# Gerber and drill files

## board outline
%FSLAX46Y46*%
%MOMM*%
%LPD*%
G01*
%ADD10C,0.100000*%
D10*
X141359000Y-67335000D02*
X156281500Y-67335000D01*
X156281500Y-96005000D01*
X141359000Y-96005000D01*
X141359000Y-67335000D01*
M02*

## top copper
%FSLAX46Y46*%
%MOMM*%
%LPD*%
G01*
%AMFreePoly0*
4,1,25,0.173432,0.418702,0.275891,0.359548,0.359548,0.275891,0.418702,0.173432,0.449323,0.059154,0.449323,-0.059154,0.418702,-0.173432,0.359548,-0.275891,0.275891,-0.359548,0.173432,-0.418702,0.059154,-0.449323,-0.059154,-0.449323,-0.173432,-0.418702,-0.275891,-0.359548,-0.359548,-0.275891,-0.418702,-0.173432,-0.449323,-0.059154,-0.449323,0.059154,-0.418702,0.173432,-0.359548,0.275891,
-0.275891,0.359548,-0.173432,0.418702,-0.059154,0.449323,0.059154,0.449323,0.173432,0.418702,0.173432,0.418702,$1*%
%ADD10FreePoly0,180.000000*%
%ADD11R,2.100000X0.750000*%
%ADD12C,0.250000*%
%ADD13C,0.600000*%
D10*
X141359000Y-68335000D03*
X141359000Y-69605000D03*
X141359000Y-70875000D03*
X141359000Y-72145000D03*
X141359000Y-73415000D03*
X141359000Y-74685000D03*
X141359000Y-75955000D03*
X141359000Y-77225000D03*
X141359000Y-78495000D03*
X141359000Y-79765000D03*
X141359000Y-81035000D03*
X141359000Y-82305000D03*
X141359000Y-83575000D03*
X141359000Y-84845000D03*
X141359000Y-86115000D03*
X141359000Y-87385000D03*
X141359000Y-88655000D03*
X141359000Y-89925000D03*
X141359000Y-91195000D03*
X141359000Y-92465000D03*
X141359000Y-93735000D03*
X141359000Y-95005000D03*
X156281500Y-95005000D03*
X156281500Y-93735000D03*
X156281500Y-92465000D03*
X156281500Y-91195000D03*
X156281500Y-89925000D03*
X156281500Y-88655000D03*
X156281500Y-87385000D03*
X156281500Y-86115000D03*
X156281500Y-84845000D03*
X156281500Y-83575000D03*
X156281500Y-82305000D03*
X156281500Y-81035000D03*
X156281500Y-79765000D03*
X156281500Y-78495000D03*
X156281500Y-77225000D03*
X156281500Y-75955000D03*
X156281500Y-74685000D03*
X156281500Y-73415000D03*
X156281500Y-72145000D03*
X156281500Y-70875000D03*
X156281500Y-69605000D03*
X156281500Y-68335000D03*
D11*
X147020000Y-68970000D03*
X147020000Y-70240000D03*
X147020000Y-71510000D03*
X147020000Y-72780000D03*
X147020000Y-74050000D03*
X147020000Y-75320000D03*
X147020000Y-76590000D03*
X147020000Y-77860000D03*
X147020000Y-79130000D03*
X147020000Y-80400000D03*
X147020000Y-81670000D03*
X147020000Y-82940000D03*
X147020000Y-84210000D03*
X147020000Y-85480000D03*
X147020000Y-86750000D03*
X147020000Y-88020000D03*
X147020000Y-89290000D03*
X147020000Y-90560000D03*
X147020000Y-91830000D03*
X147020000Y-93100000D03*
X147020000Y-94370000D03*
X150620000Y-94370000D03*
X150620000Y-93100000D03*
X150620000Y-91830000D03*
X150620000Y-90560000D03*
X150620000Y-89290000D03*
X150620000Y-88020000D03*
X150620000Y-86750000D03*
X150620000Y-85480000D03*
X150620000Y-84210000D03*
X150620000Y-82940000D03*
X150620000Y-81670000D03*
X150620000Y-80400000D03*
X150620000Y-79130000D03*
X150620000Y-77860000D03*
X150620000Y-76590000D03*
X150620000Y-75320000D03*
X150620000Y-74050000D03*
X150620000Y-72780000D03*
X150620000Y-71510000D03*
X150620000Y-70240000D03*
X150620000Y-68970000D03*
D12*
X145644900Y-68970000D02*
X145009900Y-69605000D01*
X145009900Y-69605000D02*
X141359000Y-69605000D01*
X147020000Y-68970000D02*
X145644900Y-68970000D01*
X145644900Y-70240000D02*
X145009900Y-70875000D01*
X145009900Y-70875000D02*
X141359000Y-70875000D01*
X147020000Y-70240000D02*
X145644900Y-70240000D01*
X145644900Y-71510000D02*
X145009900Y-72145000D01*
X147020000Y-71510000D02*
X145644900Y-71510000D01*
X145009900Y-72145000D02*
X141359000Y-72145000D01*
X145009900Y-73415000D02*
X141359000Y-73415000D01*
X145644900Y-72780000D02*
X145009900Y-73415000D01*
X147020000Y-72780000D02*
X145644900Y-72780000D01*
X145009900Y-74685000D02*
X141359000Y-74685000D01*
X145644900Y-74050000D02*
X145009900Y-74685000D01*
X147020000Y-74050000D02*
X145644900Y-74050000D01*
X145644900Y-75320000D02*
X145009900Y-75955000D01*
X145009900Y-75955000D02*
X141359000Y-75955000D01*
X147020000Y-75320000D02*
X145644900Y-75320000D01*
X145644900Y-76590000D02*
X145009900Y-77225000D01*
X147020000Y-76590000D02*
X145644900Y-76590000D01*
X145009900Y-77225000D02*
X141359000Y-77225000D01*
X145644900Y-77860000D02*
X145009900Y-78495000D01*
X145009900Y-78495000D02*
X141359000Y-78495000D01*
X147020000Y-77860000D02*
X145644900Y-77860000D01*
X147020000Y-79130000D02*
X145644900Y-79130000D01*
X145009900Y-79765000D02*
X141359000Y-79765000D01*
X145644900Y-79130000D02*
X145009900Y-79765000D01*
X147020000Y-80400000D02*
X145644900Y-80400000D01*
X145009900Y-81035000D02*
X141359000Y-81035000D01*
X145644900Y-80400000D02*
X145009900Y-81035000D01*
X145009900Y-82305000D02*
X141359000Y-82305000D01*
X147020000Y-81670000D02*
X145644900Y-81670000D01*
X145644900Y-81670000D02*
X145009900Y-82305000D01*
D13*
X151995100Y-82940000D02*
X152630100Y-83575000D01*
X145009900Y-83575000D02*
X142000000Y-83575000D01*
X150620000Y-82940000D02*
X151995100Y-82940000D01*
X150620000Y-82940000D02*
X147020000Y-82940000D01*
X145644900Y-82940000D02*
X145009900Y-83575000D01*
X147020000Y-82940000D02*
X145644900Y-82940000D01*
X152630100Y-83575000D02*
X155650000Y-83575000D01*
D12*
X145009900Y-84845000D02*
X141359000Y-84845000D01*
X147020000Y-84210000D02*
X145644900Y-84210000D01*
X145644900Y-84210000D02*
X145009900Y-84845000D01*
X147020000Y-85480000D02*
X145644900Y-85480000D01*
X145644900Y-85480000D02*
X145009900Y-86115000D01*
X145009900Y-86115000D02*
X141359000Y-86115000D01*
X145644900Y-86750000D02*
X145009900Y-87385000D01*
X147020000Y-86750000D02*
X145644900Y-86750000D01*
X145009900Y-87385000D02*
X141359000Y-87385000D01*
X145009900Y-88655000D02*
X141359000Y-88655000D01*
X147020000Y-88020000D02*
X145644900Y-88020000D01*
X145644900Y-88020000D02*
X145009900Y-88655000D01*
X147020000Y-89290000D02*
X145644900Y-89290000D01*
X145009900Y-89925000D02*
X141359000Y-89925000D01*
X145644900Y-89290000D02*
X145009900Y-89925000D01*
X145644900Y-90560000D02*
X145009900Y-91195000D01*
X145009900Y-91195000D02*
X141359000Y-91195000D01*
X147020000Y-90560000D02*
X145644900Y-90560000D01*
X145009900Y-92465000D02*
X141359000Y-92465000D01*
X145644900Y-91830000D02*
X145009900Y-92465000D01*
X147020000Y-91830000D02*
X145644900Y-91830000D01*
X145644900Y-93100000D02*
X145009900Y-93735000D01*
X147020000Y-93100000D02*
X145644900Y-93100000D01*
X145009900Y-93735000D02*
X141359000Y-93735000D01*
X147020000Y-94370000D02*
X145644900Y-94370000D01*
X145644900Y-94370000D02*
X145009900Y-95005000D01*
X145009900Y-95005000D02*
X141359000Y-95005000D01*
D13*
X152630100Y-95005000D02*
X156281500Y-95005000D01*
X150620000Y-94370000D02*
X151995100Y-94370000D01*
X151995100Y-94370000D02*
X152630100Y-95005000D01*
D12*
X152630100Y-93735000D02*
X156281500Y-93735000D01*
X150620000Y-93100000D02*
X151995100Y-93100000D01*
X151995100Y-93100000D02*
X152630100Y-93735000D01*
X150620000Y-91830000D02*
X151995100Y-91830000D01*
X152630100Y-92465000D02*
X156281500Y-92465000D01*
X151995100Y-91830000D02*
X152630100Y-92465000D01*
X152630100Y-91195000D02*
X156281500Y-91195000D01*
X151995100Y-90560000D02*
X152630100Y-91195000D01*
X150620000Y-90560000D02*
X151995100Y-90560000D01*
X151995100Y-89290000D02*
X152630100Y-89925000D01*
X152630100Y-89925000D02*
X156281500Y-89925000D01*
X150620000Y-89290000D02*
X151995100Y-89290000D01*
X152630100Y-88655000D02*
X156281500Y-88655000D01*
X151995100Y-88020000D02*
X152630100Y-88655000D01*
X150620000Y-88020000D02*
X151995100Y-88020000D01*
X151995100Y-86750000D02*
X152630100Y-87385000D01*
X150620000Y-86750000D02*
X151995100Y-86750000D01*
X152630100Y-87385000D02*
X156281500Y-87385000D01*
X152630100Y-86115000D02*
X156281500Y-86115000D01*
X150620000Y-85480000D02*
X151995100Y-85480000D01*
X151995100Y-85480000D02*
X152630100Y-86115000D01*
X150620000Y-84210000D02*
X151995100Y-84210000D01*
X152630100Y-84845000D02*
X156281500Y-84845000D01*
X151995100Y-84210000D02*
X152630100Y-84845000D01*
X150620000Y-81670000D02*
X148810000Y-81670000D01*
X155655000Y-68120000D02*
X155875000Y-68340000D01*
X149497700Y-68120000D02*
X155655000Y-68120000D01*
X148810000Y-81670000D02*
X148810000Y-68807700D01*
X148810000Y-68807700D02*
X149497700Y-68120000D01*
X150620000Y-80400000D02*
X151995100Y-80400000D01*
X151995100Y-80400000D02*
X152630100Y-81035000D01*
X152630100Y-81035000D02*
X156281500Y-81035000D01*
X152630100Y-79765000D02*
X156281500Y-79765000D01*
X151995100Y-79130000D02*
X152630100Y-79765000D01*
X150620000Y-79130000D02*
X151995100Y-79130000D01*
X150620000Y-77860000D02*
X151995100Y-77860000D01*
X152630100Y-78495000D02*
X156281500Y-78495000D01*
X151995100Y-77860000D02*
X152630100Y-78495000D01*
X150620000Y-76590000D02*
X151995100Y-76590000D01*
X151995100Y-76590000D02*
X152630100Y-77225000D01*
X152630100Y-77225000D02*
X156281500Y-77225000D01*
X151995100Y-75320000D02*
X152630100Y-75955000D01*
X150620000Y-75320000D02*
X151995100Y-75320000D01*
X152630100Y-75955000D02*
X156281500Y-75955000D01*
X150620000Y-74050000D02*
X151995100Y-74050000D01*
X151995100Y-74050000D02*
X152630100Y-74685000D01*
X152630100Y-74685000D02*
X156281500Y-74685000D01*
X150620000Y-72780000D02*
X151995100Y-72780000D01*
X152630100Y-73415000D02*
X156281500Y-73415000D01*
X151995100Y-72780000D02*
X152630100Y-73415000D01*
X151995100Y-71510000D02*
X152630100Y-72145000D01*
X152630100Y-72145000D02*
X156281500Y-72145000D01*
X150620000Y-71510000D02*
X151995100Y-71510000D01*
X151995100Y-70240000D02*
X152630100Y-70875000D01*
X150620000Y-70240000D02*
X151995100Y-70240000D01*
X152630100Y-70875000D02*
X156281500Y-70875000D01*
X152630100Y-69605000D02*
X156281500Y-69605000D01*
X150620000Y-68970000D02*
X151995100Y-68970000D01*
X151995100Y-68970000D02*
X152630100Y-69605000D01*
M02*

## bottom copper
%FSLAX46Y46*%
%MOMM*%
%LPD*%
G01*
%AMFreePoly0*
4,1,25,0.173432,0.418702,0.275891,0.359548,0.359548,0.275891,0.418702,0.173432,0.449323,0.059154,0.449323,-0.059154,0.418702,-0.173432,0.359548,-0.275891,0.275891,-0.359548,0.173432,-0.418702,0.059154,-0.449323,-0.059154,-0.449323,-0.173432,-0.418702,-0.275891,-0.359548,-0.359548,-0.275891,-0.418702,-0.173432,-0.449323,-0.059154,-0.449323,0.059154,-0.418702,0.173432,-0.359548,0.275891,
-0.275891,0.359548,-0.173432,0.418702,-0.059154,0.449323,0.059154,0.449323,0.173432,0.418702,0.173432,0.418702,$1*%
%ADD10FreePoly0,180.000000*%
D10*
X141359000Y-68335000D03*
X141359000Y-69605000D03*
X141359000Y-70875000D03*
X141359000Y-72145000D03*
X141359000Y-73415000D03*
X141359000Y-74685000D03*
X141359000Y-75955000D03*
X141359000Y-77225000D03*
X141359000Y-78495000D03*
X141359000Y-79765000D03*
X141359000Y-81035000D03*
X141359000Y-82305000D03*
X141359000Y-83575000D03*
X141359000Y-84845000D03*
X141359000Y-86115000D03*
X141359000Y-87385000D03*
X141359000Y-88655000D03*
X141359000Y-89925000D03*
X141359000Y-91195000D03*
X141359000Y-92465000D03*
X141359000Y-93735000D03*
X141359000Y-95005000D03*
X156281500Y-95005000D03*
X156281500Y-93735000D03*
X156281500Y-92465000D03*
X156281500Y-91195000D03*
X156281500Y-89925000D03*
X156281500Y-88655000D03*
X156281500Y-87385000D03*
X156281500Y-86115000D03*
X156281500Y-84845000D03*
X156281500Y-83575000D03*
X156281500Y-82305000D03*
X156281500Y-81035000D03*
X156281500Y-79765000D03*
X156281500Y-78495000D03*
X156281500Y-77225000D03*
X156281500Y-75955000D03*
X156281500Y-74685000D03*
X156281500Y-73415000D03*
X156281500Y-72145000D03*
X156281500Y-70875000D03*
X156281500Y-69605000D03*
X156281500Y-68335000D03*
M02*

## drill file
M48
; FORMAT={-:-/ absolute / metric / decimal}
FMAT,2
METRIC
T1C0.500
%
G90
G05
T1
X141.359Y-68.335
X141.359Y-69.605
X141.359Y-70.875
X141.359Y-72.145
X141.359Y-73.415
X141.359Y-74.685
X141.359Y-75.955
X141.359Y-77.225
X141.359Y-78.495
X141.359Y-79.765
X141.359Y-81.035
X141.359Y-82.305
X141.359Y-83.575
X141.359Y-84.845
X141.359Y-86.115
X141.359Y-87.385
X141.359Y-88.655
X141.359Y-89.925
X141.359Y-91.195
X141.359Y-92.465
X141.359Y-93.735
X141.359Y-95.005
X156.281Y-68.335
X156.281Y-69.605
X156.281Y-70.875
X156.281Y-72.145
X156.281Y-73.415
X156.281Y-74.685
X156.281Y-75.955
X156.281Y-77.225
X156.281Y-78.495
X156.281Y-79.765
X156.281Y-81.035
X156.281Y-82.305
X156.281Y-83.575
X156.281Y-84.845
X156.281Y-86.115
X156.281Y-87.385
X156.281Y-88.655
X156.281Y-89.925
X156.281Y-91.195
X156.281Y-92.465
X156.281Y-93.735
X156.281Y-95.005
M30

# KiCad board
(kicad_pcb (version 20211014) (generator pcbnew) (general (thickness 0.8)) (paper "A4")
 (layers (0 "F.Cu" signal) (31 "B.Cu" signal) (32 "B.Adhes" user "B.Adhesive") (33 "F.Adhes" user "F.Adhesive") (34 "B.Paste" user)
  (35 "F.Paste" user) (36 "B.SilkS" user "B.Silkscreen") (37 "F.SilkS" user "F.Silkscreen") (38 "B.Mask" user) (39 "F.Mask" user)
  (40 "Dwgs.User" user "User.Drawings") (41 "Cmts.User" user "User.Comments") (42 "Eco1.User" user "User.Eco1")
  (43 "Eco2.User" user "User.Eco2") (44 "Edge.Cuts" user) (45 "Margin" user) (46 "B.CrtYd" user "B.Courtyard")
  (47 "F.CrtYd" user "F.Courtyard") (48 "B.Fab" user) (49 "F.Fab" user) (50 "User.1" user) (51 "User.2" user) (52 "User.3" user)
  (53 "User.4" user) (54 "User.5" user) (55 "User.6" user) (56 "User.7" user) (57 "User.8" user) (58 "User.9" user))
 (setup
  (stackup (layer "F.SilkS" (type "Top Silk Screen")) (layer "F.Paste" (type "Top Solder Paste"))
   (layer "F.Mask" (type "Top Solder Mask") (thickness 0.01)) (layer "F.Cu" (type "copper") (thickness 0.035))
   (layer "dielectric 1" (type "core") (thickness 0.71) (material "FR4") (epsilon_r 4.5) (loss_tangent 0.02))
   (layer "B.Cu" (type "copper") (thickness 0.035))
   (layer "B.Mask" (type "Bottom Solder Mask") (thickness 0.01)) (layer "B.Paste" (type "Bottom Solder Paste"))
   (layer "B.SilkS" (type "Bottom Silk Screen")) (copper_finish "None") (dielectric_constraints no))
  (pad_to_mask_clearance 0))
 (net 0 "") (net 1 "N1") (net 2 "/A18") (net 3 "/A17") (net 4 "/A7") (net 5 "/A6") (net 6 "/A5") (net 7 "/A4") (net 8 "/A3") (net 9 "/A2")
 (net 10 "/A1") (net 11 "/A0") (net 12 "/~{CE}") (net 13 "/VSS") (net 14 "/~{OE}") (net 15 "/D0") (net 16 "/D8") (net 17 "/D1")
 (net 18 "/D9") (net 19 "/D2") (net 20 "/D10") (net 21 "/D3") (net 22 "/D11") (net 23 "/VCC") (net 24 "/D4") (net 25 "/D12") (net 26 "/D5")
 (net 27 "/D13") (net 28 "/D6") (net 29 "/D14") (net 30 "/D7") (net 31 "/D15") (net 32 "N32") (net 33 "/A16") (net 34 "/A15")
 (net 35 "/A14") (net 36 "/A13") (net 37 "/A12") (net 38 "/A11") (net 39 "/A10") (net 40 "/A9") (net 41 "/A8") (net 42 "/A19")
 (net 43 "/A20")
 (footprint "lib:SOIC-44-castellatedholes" (layer "F.Cu") (at 148.82 81.67)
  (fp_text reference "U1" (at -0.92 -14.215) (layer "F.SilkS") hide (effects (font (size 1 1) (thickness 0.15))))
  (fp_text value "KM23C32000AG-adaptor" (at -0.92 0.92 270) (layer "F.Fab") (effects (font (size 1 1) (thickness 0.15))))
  (pad "1" thru_hole custom (at -7.461 -13.335 180) (size 0.9064 0.9064) (drill 0.5) (layers *.Cu *.Mask) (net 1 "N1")
   (solder_mask_margin 0.0762) (options (clearance outline) (anchor circle)) (primitives))
  (pad "2" thru_hole custom (at -7.461 -12.065 180) (size 0.9064 0.9064) (drill 0.5) (layers *.Cu *.Mask) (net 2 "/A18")
   (solder_mask_margin 0.0762) (options (clearance outline) (anchor circle)) (primitives))
  (pad "3" thru_hole custom (at -7.461 -10.795 180) (size 0.9064 0.9064) (drill 0.5) (layers *.Cu *.Mask) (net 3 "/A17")
   (solder_mask_margin 0.0762) (options (clearance outline) (anchor circle)) (primitives))
  (pad "4" thru_hole custom (at -7.461 -9.525 180) (size 0.9064 0.9064) (drill 0.5) (layers *.Cu *.Mask) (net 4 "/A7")
   (solder_mask_margin 0.0762) (options (clearance outline) (anchor circle)) (primitives))
  (pad "5" thru_hole custom (at -7.461 -8.255 180) (size 0.9064 0.9064) (drill 0.5) (layers *.Cu *.Mask) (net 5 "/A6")
   (solder_mask_margin 0.0762) (options (clearance outline) (anchor circle)) (primitives))
  (pad "6" thru_hole custom (at -7.461 -6.985 180) (size 0.9064 0.9064) (drill 0.5) (layers *.Cu *.Mask) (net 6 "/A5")
   (solder_mask_margin 0.0762) (options (clearance outline) (anchor circle)) (primitives))
  (pad "7" thru_hole custom (at -7.461 -5.715 180) (size 0.9064 0.9064) (drill 0.5) (layers *.Cu *.Mask) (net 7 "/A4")
   (solder_mask_margin 0.0762) (options (clearance outline) (anchor circle)) (primitives))
  (pad "8" thru_hole custom (at -7.461 -4.445 180) (size 0.9064 0.9064) (drill 0.5) (layers *.Cu *.Mask) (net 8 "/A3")
   (solder_mask_margin 0.0762) (options (clearance outline) (anchor circle)) (primitives))
  (pad "9" thru_hole custom (at -7.461 -3.175 180) (size 0.9064 0.9064) (drill 0.5) (layers *.Cu *.Mask) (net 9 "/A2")
   (solder_mask_margin 0.0762) (options (clearance outline) (anchor circle)) (primitives))
  (pad "10" thru_hole custom (at -7.461 -1.905 180) (size 0.9064 0.9064) (drill 0.5) (layers *.Cu *.Mask) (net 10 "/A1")
   (solder_mask_margin 0.0762) (options (clearance outline) (anchor circle)) (primitives))
  (pad "11" thru_hole custom (at -7.461 -0.635 180) (size 0.9064 0.9064) (drill 0.5) (layers *.Cu *.Mask) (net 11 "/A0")
   (solder_mask_margin 0.0762) (options (clearance outline) (anchor circle)) (primitives))
  (pad "12" thru_hole custom (at -7.461 0.635 180) (size 0.9064 0.9064) (drill 0.5) (layers *.Cu *.Mask) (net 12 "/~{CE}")
   (solder_mask_margin 0.0762) (options (clearance outline) (anchor circle)) (primitives))
  (pad "13" thru_hole custom (at -7.461 1.905 180) (size 0.9064 0.9064) (drill 0.5) (layers *.Cu *.Mask) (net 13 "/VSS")
   (solder_mask_margin 0.0762) (options (clearance outline) (anchor circle)) (primitives))
  (pad "14" thru_hole custom (at -7.461 3.175 180) (size 0.9064 0.9064) (drill 0.5) (layers *.Cu *.Mask) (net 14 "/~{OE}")
   (solder_mask_margin 0.0762) (options (clearance outline) (anchor circle)) (primitives))
  (pad "15" thru_hole custom (at -7.461 4.445 180) (size 0.9064 0.9064) (drill 0.5) (layers *.Cu *.Mask) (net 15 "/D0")
   (solder_mask_margin 0.0762) (options (clearance outline) (anchor circle)) (primitives))
  (pad "16" thru_hole custom (at -7.461 5.715 180) (size 0.9064 0.9064) (drill 0.5) (layers *.Cu *.Mask) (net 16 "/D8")
   (solder_mask_margin 0.0762) (options (clearance outline) (anchor circle)) (primitives))
  (pad "17" thru_hole custom (at -7.461 6.985 180) (size 0.9064 0.9064) (drill 0.5) (layers *.Cu *.Mask) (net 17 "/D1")
   (solder_mask_margin 0.0762) (options (clearance outline) (anchor circle)) (primitives))
  (pad "18" thru_hole custom (at -7.461 8.255 180) (size 0.9064 0.9064) (drill 0.5) (layers *.Cu *.Mask) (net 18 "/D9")
   (solder_mask_margin 0.0762) (options (clearance outline) (anchor circle)) (primitives))
  (pad "19" thru_hole custom (at -7.461 9.525 180) (size 0.9064 0.9064) (drill 0.5) (layers *.Cu *.Mask) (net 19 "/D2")
   (solder_mask_margin 0.0762) (options (clearance outline) (anchor circle)) (primitives))
  (pad "20" thru_hole custom (at -7.461 10.795 180) (size 0.9064 0.9064) (drill 0.5) (layers *.Cu *.Mask) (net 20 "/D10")
   (solder_mask_margin 0.0762) (options (clearance outline) (anchor circle)) (primitives))
  (pad "21" thru_hole custom (at -7.461 12.065 180) (size 0.9064 0.9064) (drill 0.5) (layers *.Cu *.Mask) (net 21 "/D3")
   (solder_mask_margin 0.0762) (options (clearance outline) (anchor circle)) (primitives))
  (pad "22" thru_hole custom (at -7.461 13.335 180) (size 0.9064 0.9064) (drill 0.5) (layers *.Cu *.Mask) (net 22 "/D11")
   (solder_mask_margin 0.0762) (options (clearance outline) (anchor circle)) (primitives))
  (pad "23" thru_hole custom (at 7.4615 13.335 180) (size 0.9064 0.9064) (drill 0.5) (layers *.Cu *.Mask) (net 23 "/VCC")
   (solder_mask_margin 0.0762) (options (clearance outline) (anchor circle)) (primitives))
  (pad "24" thru_hole custom (at 7.4615 12.065 180) (size 0.9064 0.9064) (drill 0.5) (layers *.Cu *.Mask) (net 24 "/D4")
   (solder_mask_margin 0.0762) (options (clearance outline) (anchor circle)) (primitives))
  (pad "25" thru_hole custom (at 7.4615 10.795 180) (size 0.9064 0.9064) (drill 0.5) (layers *.Cu *.Mask) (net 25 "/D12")
   (solder_mask_margin 0.0762) (options (clearance outline) (anchor circle)) (primitives))
  (pad "26" thru_hole custom (at 7.4615 9.525 180) (size 0.9064 0.9064) (drill 0.5) (layers *.Cu *.Mask) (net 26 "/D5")
   (solder_mask_margin 0.0762) (options (clearance outline) (anchor circle)) (primitives))
  (pad "27" thru_hole custom (at 7.4615 8.255 180) (size 0.9064 0.9064) (drill 0.5) (layers *.Cu *.Mask) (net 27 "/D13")
   (solder_mask_margin 0.0762) (options (clearance outline) (anchor circle)) (primitives))
  (pad "28" thru_hole custom (at 7.4615 6.985 180) (size 0.9064 0.9064) (drill 0.5) (layers *.Cu *.Mask) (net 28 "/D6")
   (solder_mask_margin 0.0762) (options (clearance outline) (anchor circle)) (primitives))
  (pad "29" thru_hole custom (at 7.4615 5.715 180) (size 0.9064 0.9064) (drill 0.5) (layers *.Cu *.Mask) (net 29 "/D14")
   (solder_mask_margin 0.0762) (options (clearance outline) (anchor circle)) (primitives))
  (pad "30" thru_hole custom (at 7.4615 4.445 180) (size 0.9064 0.9064) (drill 0.5) (layers *.Cu *.Mask) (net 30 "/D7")
   (solder_mask_margin 0.0762) (options (clearance outline) (anchor circle)) (primitives))
  (pad "31" thru_hole custom (at 7.4615 3.175 180) (size 0.9064 0.9064) (drill 0.5) (layers *.Cu *.Mask) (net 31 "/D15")
   (solder_mask_margin 0.0762) (options (clearance outline) (anchor circle)) (primitives))
  (pad "32" thru_hole custom (at 7.4615 1.905 180) (size 0.9064 0.9064) (drill 0.5) (layers *.Cu *.Mask) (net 13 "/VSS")
   (solder_mask_margin 0.0762) (options (clearance outline) (anchor circle)) (primitives))
  (pad "33" thru_hole custom (at 7.4615 0.635 180) (size 0.9064 0.9064) (drill 0.5) (layers *.Cu *.Mask) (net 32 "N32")
   (solder_mask_margin 0.0762) (options (clearance outline) (anchor circle)) (primitives))
  (pad "34" thru_hole custom (at 7.4615 -0.635 180) (size 0.9064 0.9064) (drill 0.5) (layers *.Cu *.Mask) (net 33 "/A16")
   (solder_mask_margin 0.0762) (options (clearance outline) (anchor circle)) (primitives))
  (pad "35" thru_hole custom (at 7.4615 -1.905 180) (size 0.9064 0.9064) (drill 0.5) (layers *.Cu *.Mask) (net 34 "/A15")
   (solder_mask_margin 0.0762) (options (clearance outline) (anchor circle)) (primitives))
  (pad "36" thru_hole custom (at 7.4615 -3.175 180) (size 0.9064 0.9064) (drill 0.5) (layers *.Cu *.Mask) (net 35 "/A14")
   (solder_mask_margin 0.0762) (options (clearance outline) (anchor circle)) (primitives))
  (pad "37" thru_hole custom (at 7.4615 -4.445 180) (size 0.9064 0.9064) (drill 0.5) (layers *.Cu *.Mask) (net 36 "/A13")
   (solder_mask_margin 0.0762) (options (clearance outline) (anchor circle)) (primitives))
  (pad "38" thru_hole custom (at 7.4615 -5.715 180) (size 0.9064 0.9064) (drill 0.5) (layers *.Cu *.Mask) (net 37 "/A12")
   (solder_mask_margin 0.0762) (options (clearance outline) (anchor circle)) (primitives))
  (pad "39" thru_hole custom (at 7.4615 -6.985 180) (size 0.9064 0.9064) (drill 0.5) (layers *.Cu *.Mask) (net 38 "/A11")
   (solder_mask_margin 0.0762) (options (clearance outline) (anchor circle)) (primitives))
  (pad "40" thru_hole custom (at 7.4615 -8.255 180) (size 0.9064 0.9064) (drill 0.5) (layers *.Cu *.Mask) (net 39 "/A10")
   (solder_mask_margin 0.0762) (options (clearance outline) (anchor circle)) (primitives))
  (pad "41" thru_hole custom (at 7.4615 -9.525 180) (size 0.9064 0.9064) (drill 0.5) (layers *.Cu *.Mask) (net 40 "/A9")
   (solder_mask_margin 0.0762) (options (clearance outline) (anchor circle)) (primitives))
  (pad "42" thru_hole custom (at 7.4615 -10.795 180) (size 0.9064 0.9064) (drill 0.5) (layers *.Cu *.Mask) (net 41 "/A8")
   (solder_mask_margin 0.0762) (options (clearance outline) (anchor circle)) (primitives))
  (pad "43" thru_hole custom (at 7.4615 -12.065 180) (size 0.9064 0.9064) (drill 0.5) (layers *.Cu *.Mask) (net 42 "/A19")
   (solder_mask_margin 0.0762) (options (clearance outline) (anchor circle)) (primitives))
  (pad "44" thru_hole custom (at 7.4615 -13.335 180) (size 0.9064 0.9064) (drill 0.5) (layers *.Cu *.Mask) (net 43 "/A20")
   (solder_mask_margin 0.0762) (options (clearance outline) (anchor circle)) (primitives)))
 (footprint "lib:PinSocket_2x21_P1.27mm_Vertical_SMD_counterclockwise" (layer "F.Cu") (at 148.82 81.67)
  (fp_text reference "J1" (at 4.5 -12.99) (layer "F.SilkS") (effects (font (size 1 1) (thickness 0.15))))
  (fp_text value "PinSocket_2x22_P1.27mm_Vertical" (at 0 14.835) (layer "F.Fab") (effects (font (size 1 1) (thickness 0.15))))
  (pad "1" smd rect (at -1.8 -12.7) (size 2.1 0.75) (layers "F.Cu" "F.Paste" "F.Mask") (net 2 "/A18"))
  (pad "2" smd rect (at -1.8 -11.43) (size 2.1 0.75) (layers "F.Cu" "F.Paste" "F.Mask") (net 3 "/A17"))
  (pad "3" smd rect (at -1.8 -10.16) (size 2.1 0.75) (layers "F.Cu" "F.Paste" "F.Mask") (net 4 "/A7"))
  (pad "4" smd rect (at -1.8 -8.89) (size 2.1 0.75) (layers "F.Cu" "F.Paste" "F.Mask") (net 5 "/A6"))
  (pad "5" smd rect (at -1.8 -7.62) (size 2.1 0.75) (layers "F.Cu" "F.Paste" "F.Mask") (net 6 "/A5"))
  (pad "6" smd rect (at -1.8 -6.35) (size 2.1 0.75) (layers "F.Cu" "F.Paste" "F.Mask") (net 7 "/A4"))
  (pad "7" smd rect (at -1.8 -5.08) (size 2.1 0.75) (layers "F.Cu" "F.Paste" "F.Mask") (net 8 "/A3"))
  (pad "8" smd rect (at -1.8 -3.81) (size 2.1 0.75) (layers "F.Cu" "F.Paste" "F.Mask") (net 9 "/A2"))
  (pad "9" smd rect (at -1.8 -2.54) (size 2.1 0.75) (layers "F.Cu" "F.Paste" "F.Mask") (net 10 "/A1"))
  (pad "10" smd rect (at -1.8 -1.27) (size 2.1 0.75) (layers "F.Cu" "F.Paste" "F.Mask") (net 11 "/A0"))
  (pad "11" smd rect (at -1.8 0) (size 2.1 0.75) (layers "F.Cu" "F.Paste" "F.Mask") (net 12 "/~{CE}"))
  (pad "12" smd rect (at -1.8 1.27) (size 2.1 0.75) (layers "F.Cu" "F.Paste" "F.Mask") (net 13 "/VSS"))
  (pad "13" smd rect (at -1.8 2.54) (size 2.1 0.75) (layers "F.Cu" "F.Paste" "F.Mask") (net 14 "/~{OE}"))
  (pad "14" smd rect (at -1.8 3.81) (size 2.1 0.75) (layers "F.Cu" "F.Paste" "F.Mask") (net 15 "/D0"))
  (pad "15" smd rect (at -1.8 5.08) (size 2.1 0.75) (layers "F.Cu" "F.Paste" "F.Mask") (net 16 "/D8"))
  (pad "16" smd rect (at -1.8 6.35) (size 2.1 0.75) (layers "F.Cu" "F.Paste" "F.Mask") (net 17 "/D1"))
  (pad "17" smd rect (at -1.8 7.62) (size 2.1 0.75) (layers "F.Cu" "F.Paste" "F.Mask") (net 18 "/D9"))
  (pad "18" smd rect (at -1.8 8.89) (size 2.1 0.75) (layers "F.Cu" "F.Paste" "F.Mask") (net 19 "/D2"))
  (pad "19" smd rect (at -1.8 10.16) (size 2.1 0.75) (layers "F.Cu" "F.Paste" "F.Mask") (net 20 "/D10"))
  (pad "20" smd rect (at -1.8 11.43) (size 2.1 0.75) (layers "F.Cu" "F.Paste" "F.Mask") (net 21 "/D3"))
  (pad "21" smd rect (at -1.8 12.7) (size 2.1 0.75) (layers "F.Cu" "F.Paste" "F.Mask") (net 22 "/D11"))
  (pad "22" smd rect (at 1.8 12.7) (size 2.1 0.75) (layers "F.Cu" "F.Paste" "F.Mask") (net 23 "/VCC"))
  (pad "23" smd rect (at 1.8 11.43) (size 2.1 0.75) (layers "F.Cu" "F.Paste" "F.Mask") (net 24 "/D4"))
  (pad "24" smd rect (at 1.8 10.16) (size 2.1 0.75) (layers "F.Cu" "F.Paste" "F.Mask") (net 25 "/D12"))
  (pad "25" smd rect (at 1.8 8.89) (size 2.1 0.75) (layers "F.Cu" "F.Paste" "F.Mask") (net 26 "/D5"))
  (pad "26" smd rect (at 1.8 7.62) (size 2.1 0.75) (layers "F.Cu" "F.Paste" "F.Mask") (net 27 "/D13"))
  (pad "27" smd rect (at 1.8 6.35) (size 2.1 0.75) (layers "F.Cu" "F.Paste" "F.Mask") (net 28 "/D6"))
  (pad "28" smd rect (at 1.8 5.08) (size 2.1 0.75) (layers "F.Cu" "F.Paste" "F.Mask") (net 29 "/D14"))
  (pad "29" smd rect (at 1.8 3.81) (size 2.1 0.75) (layers "F.Cu" "F.Paste" "F.Mask") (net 30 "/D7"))
  (pad "30" smd rect (at 1.8 2.54) (size 2.1 0.75) (layers "F.Cu" "F.Paste" "F.Mask") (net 31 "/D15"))
  (pad "31" smd rect (at 1.8 1.27) (size 2.1 0.75) (layers "F.Cu" "F.Paste" "F.Mask") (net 13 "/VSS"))
  (pad "32" smd rect (at 1.8 0) (size 2.1 0.75) (layers "F.Cu" "F.Paste" "F.Mask") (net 43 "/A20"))
  (pad "33" smd rect (at 1.8 -1.27) (size 2.1 0.75) (layers "F.Cu" "F.Paste" "F.Mask") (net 33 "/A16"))
  (pad "34" smd rect (at 1.8 -2.54) (size 2.1 0.75) (layers "F.Cu" "F.Paste" "F.Mask") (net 34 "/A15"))
  (pad "35" smd rect (at 1.8 -3.81) (size 2.1 0.75) (layers "F.Cu" "F.Paste" "F.Mask") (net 35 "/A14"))
  (pad "36" smd rect (at 1.8 -5.08) (size 2.1 0.75) (layers "F.Cu" "F.Paste" "F.Mask") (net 36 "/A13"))
  (pad "37" smd rect (at 1.8 -6.35) (size 2.1 0.75) (layers "F.Cu" "F.Paste" "F.Mask") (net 37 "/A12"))
  (pad "38" smd rect (at 1.8 -7.62) (size 2.1 0.75) (layers "F.Cu" "F.Paste" "F.Mask") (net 38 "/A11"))
  (pad "39" smd rect (at 1.8 -8.89) (size 2.1 0.75) (layers "F.Cu" "F.Paste" "F.Mask") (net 39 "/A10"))
  (pad "40" smd rect (at 1.8 -10.16) (size 2.1 0.75) (layers "F.Cu" "F.Paste" "F.Mask") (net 40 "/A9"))
  (pad "41" smd rect (at 1.8 -11.43) (size 2.1 0.75) (layers "F.Cu" "F.Paste" "F.Mask") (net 41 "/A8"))
  (pad "42" smd rect (at 1.8 -12.7) (size 2.1 0.75) (layers "F.Cu" "F.Paste" "F.Mask") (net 42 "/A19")))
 (gr_rect (start 141.359 67.335) (end 156.2815 96.005) (layer "Edge.Cuts") (width 0.1) (fill none))
 (segment (start 145.6449 68.97) (end 145.0099 69.605) (width 0.25) (layer "F.Cu") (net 2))
 (segment (start 145.0099 69.605) (end 141.359 69.605) (width 0.25) (layer "F.Cu") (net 2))
 (segment (start 147.02 68.97) (end 145.6449 68.97) (width 0.25) (layer "F.Cu") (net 2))
 (segment (start 145.6449 70.24) (end 145.0099 70.875) (width 0.25) (layer "F.Cu") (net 3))
 (segment (start 145.0099 70.875) (end 141.359 70.875) (width 0.25) (layer "F.Cu") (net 3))
 (segment (start 147.02 70.24) (end 145.6449 70.24) (width 0.25) (layer "F.Cu") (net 3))
 (segment (start 145.6449 71.51) (end 145.0099 72.145) (width 0.25) (layer "F.Cu") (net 4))
 (segment (start 147.02 71.51) (end 145.6449 71.51) (width 0.25) (layer "F.Cu") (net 4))
 (segment (start 145.0099 72.145) (end 141.359 72.145) (width 0.25) (layer "F.Cu") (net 4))
 (segment (start 145.0099 73.415) (end 141.359 73.415) (width 0.25) (layer "F.Cu") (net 5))
 (segment (start 145.6449 72.78) (end 145.0099 73.415) (width 0.25) (layer "F.Cu") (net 5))
 (segment (start 147.02 72.78) (end 145.6449 72.78) (width 0.25) (layer "F.Cu") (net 5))
 (segment (start 145.0099 74.685) (end 141.359 74.685) (width 0.25) (layer "F.Cu") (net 6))
 (segment (start 145.6449 74.05) (end 145.0099 74.685) (width 0.25) (layer "F.Cu") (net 6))
 (segment (start 147.02 74.05) (end 145.6449 74.05) (width 0.25) (layer "F.Cu") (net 6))
 (segment (start 145.6449 75.32) (end 145.0099 75.955) (width 0.25) (layer "F.Cu") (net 7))
 (segment (start 145.0099 75.955) (end 141.359 75.955) (width 0.25) (layer "F.Cu") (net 7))
 (segment (start 147.02 75.32) (end 145.6449 75.32) (width 0.25) (layer "F.Cu") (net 7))
 (segment (start 145.6449 76.59) (end 145.0099 77.225) (width 0.25) (layer "F.Cu") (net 8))
 (segment (start 147.02 76.59) (end 145.6449 76.59) (width 0.25) (layer "F.Cu") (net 8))
 (segment (start 145.0099 77.225) (end 141.359 77.225) (width 0.25) (layer "F.Cu") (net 8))
 (segment (start 145.6449 77.86) (end 145.0099 78.495) (width 0.25) (layer "F.Cu") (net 9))
 (segment (start 145.0099 78.495) (end 141.359 78.495) (width 0.25) (layer "F.Cu") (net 9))
 (segment (start 147.02 77.86) (end 145.6449 77.86) (width 0.25) (layer "F.Cu") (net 9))
 (segment (start 147.02 79.13) (end 145.6449 79.13) (width 0.25) (layer "F.Cu") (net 10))
 (segment (start 145.0099 79.765) (end 141.359 79.765) (width 0.25) (layer "F.Cu") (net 10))
 (segment (start 145.6449 79.13) (end 145.0099 79.765) (width 0.25) (layer "F.Cu") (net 10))
 (segment (start 147.02 80.4) (end 145.6449 80.4) (width 0.25) (layer "F.Cu") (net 11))
 (segment (start 145.0099 81.035) (end 141.359 81.035) (width 0.25) (layer "F.Cu") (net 11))
 (segment (start 145.6449 80.4) (end 145.0099 81.035) (width 0.25) (layer "F.Cu") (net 11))
 (segment (start 145.0099 82.305) (end 141.359 82.305) (width 0.25) (layer "F.Cu") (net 12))
 (segment (start 147.02 81.67) (end 145.6449 81.67) (width 0.25) (layer "F.Cu") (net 12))
 (segment (start 145.6449 81.67) (end 145.0099 82.305) (width 0.25) (layer "F.Cu") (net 12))
 (segment (start 151.9951 82.94) (end 152.6301 83.575) (width 0.6) (layer "F.Cu") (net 13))
 (segment (start 145.0099 83.575) (end 142 83.575) (width 0.6) (layer "F.Cu") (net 13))
 (segment (start 150.62 82.94) (end 151.9951 82.94) (width 0.6) (layer "F.Cu") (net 13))
 (segment (start 150.62 82.94) (end 147.02 82.94) (width 0.6) (layer "F.Cu") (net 13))
 (segment (start 145.6449 82.94) (end 145.0099 83.575) (width 0.6) (layer "F.Cu") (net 13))
 (segment (start 147.02 82.94) (end 145.6449 82.94) (width 0.6) (layer "F.Cu") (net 13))
 (segment (start 152.6301 83.575) (end 155.65 83.575) (width 0.6) (layer "F.Cu") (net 13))
 (segment (start 145.0099 84.845) (end 141.359 84.845) (width 0.25) (layer "F.Cu") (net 14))
 (segment (start 147.02 84.21) (end 145.6449 84.21) (width 0.25) (layer "F.Cu") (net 14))
 (segment (start 145.6449 84.21) (end 145.0099 84.845) (width 0.25) (layer "F.Cu") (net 14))
 (segment (start 147.02 85.48) (end 145.6449 85.48) (width 0.25) (layer "F.Cu") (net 15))
 (segment (start 145.6449 85.48) (end 145.0099 86.115) (width 0.25) (layer "F.Cu") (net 15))
 (segment (start 145.0099 86.115) (end 141.359 86.115) (width 0.25) (layer "F.Cu") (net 15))
 (segment (start 145.6449 86.75) (end 145.0099 87.385) (width 0.25) (layer "F.Cu") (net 16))
 (segment (start 147.02 86.75) (end 145.6449 86.75) (width 0.25) (layer "F.Cu") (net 16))
 (segment (start 145.0099 87.385) (end 141.359 87.385) (width 0.25) (layer "F.Cu") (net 16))
 (segment (start 145.0099 88.655) (end 141.359 88.655) (width 0.25) (layer "F.Cu") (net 17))
 (segment (start 147.02 88.02) (end 145.6449 88.02) (width 0.25) (layer "F.Cu") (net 17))
 (segment (start 145.6449 88.02) (end 145.0099 88.655) (width 0.25) (layer "F.Cu") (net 17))
 (segment (start 147.02 89.29) (end 145.6449 89.29) (width 0.25) (layer "F.Cu") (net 18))
 (segment (start 145.0099 89.925) (end 141.359 89.925) (width 0.25) (layer "F.Cu") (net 18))
 (segment (start 145.6449 89.29) (end 145.0099 89.925) (width 0.25) (layer "F.Cu") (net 18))
 (segment (start 145.6449 90.56) (end 145.0099 91.195) (width 0.25) (layer "F.Cu") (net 19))
 (segment (start 145.0099 91.195) (end 141.359 91.195) (width 0.25) (layer "F.Cu") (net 19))
 (segment (start 147.02 90.56) (end 145.6449 90.56) (width 0.25) (layer "F.Cu") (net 19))
 (segment (start 145.0099 92.465) (end 141.359 92.465) (width 0.25) (layer "F.Cu") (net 20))
 (segment (start 145.6449 91.83) (end 145.0099 92.465) (width 0.25) (layer "F.Cu") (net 20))
 (segment (start 147.02 91.83) (end 145.6449 91.83) (width 0.25) (layer "F.Cu") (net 20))
 (segment (start 145.6449 93.1) (end 145.0099 93.735) (width 0.25) (layer "F.Cu") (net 21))
 (segment (start 147.02 93.1) (end 145.6449 93.1) (width 0.25) (layer "F.Cu") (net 21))
 (segment (start 145.0099 93.735) (end 141.359 93.735) (width 0.25) (layer "F.Cu") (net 21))
 (segment (start 147.02 94.37) (end 145.6449 94.37) (width 0.25) (layer "F.Cu") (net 22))
 (segment (start 145.6449 94.37) (end 145.0099 95.005) (width 0.25) (layer "F.Cu") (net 22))
 (segment (start 145.0099 95.005) (end 141.359 95.005) (width 0.25) (layer "F.Cu") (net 22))
 (segment (start 152.6301 95.005) (end 156.2815 95.005) (width 0.6) (layer "F.Cu") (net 23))
 (segment (start 150.62 94.37) (end 151.9951 94.37) (width 0.6) (layer "F.Cu") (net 23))
 (segment (start 151.9951 94.37) (end 152.6301 95.005) (width 0.6) (layer "F.Cu") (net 23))
 (segment (start 152.6301 93.735) (end 156.2815 93.735) (width 0.25) (layer "F.Cu") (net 24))
 (segment (start 150.62 93.1) (end 151.9951 93.1) (width 0.25) (layer "F.Cu") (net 24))
 (segment (start 151.9951 93.1) (end 152.6301 93.735) (width 0.25) (layer "F.Cu") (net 24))
 (segment (start 150.62 91.83) (end 151.9951 91.83) (width 0.25) (layer "F.Cu") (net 25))
 (segment (start 152.6301 92.465) (end 156.2815 92.465) (width 0.25) (layer "F.Cu") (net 25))
 (segment (start 151.9951 91.83) (end 152.6301 92.465) (width 0.25) (layer "F.Cu") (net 25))
 (segment (start 152.6301 91.195) (end 156.2815 91.195) (width 0.25) (layer "F.Cu") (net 26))
 (segment (start 151.9951 90.56) (end 152.6301 91.195) (width 0.25) (layer "F.Cu") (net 26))
 (segment (start 150.62 90.56) (end 151.9951 90.56) (width 0.25) (layer "F.Cu") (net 26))
 (segment (start 151.9951 89.29) (end 152.6301 89.925) (width 0.25) (layer "F.Cu") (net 27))
 (segment (start 152.6301 89.925) (end 156.2815 89.925) (width 0.25) (layer "F.Cu") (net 27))
 (segment (start 150.62 89.29) (end 151.9951 89.29) (width 0.25) (layer "F.Cu") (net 27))
 (segment (start 152.6301 88.655) (end 156.2815 88.655) (width 0.25) (layer "F.Cu") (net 28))
 (segment (start 151.9951 88.02) (end 152.6301 88.655) (width 0.25) (layer "F.Cu") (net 28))
 (segment (start 150.62 88.02) (end 151.9951 88.02) (width 0.25) (layer "F.Cu") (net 28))
 (segment (start 151.9951 86.75) (end 152.6301 87.385) (width 0.25) (layer "F.Cu") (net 29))
 (segment (start 150.62 86.75) (end 151.9951 86.75) (width 0.25) (layer "F.Cu") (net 29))
 (segment (start 152.6301 87.385) (end 156.2815 87.385) (width 0.25) (layer "F.Cu") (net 29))
 (segment (start 152.6301 86.115) (end 156.2815 86.115) (width 0.25) (layer "F.Cu") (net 30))
 (segment (start 150.62 85.48) (end 151.9951 85.48) (width 0.25) (layer "F.Cu") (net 30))
 (segment (start 151.9951 85.48) (end 152.6301 86.115) (width 0.25) (layer "F.Cu") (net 30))
 (segment (start 150.62 84.21) (end 151.9951 84.21) (width 0.25) (layer "F.Cu") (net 31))
 (segment (start 152.6301 84.845) (end 156.2815 84.845) (width 0.25) (layer "F.Cu") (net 31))
 (segment (start 151.9951 84.21) (end 152.6301 84.845) (width 0.25) (layer "F.Cu") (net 31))
 (segment (start 150.62 81.67) (end 148.81 81.67) (width 0.25) (layer "F.Cu") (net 43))
 (segment (start 155.655 68.12) (end 155.875 68.34) (width 0.25) (layer "F.Cu") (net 43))
 (segment (start 149.4977 68.12) (end 155.655 68.12) (width 0.25) (layer "F.Cu") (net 43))
 (segment (start 148.81 81.67) (end 148.81 68.8077) (width 0.25) (layer "F.Cu") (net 43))
 (segment (start 148.81 68.8077) (end 149.4977 68.12) (width 0.25) (layer "F.Cu") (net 43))
 (segment (start 150.62 80.4) (end 151.9951 80.4) (width 0.25) (layer "F.Cu") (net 33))
 (segment (start 151.9951 80.4) (end 152.6301 81.035) (width 0.25) (layer "F.Cu") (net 33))
 (segment (start 152.6301 81.035) (end 156.2815 81.035) (width 0.25) (layer "F.Cu") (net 33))
 (segment (start 152.6301 79.765) (end 156.2815 79.765) (width 0.25) (layer "F.Cu") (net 34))
 (segment (start 151.9951 79.13) (end 152.6301 79.765) (width 0.25) (layer "F.Cu") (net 34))
 (segment (start 150.62 79.13) (end 151.9951 79.13) (width 0.25) (layer "F.Cu") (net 34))
 (segment (start 150.62 77.86) (end 151.9951 77.86) (width 0.25) (layer "F.Cu") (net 35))
 (segment (start 152.6301 78.495) (end 156.2815 78.495) (width 0.25) (layer "F.Cu") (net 35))
 (segment (start 151.9951 77.86) (end 152.6301 78.495) (width 0.25) (layer "F.Cu") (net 35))
 (segment (start 150.62 76.59) (end 151.9951 76.59) (width 0.25) (layer "F.Cu") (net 36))
 (segment (start 151.9951 76.59) (end 152.6301 77.225) (width 0.25) (layer "F.Cu") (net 36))
 (segment (start 152.6301 77.225) (end 156.2815 77.225) (width 0.25) (layer "F.Cu") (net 36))
 (segment (start 151.9951 75.32) (end 152.6301 75.955) (width 0.25) (layer "F.Cu") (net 37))
 (segment (start 150.62 75.32) (end 151.9951 75.32) (width 0.25) (layer "F.Cu") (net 37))
 (segment (start 152.6301 75.955) (end 156.2815 75.955) (width 0.25) (layer "F.Cu") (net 37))
 (segment (start 150.62 74.05) (end 151.9951 74.05) (width 0.25) (layer "F.Cu") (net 38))
 (segment (start 151.9951 74.05) (end 152.6301 74.685) (width 0.25) (layer "F.Cu") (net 38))
 (segment (start 152.6301 74.685) (end 156.2815 74.685) (width 0.25) (layer "F.Cu") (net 38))
 (segment (start 150.62 72.78) (end 151.9951 72.78) (width 0.25) (layer "F.Cu") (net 39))
 (segment (start 152.6301 73.415) (end 156.2815 73.415) (width 0.25) (layer "F.Cu") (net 39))
 (segment (start 151.9951 72.78) (end 152.6301 73.415) (width 0.25) (layer "F.Cu") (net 39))
 (segment (start 151.9951 71.51) (end 152.6301 72.145) (width 0.25) (layer "F.Cu") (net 40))
 (segment (start 152.6301 72.145) (end 156.2815 72.145) (width 0.25) (layer "F.Cu") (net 40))
 (segment (start 150.62 71.51) (end 151.9951 71.51) (width 0.25) (layer "F.Cu") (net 40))
 (segment (start 151.9951 70.24) (end 152.6301 70.875) (width 0.25) (layer "F.Cu") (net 41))
 (segment (start 150.62 70.24) (end 151.9951 70.24) (width 0.25) (layer "F.Cu") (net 41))
 (segment (start 152.6301 70.875) (end 156.2815 70.875) (width 0.25) (layer "F.Cu") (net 41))
 (segment (start 152.6301 69.605) (end 156.2815 69.605) (width 0.25) (layer "F.Cu") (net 42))
 (segment (start 150.62 68.97) (end 151.9951 68.97) (width 0.25) (layer "F.Cu") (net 42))
 (segment (start 151.9951 68.97) (end 152.6301 69.605) (width 0.25) (layer "F.Cu") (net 42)))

